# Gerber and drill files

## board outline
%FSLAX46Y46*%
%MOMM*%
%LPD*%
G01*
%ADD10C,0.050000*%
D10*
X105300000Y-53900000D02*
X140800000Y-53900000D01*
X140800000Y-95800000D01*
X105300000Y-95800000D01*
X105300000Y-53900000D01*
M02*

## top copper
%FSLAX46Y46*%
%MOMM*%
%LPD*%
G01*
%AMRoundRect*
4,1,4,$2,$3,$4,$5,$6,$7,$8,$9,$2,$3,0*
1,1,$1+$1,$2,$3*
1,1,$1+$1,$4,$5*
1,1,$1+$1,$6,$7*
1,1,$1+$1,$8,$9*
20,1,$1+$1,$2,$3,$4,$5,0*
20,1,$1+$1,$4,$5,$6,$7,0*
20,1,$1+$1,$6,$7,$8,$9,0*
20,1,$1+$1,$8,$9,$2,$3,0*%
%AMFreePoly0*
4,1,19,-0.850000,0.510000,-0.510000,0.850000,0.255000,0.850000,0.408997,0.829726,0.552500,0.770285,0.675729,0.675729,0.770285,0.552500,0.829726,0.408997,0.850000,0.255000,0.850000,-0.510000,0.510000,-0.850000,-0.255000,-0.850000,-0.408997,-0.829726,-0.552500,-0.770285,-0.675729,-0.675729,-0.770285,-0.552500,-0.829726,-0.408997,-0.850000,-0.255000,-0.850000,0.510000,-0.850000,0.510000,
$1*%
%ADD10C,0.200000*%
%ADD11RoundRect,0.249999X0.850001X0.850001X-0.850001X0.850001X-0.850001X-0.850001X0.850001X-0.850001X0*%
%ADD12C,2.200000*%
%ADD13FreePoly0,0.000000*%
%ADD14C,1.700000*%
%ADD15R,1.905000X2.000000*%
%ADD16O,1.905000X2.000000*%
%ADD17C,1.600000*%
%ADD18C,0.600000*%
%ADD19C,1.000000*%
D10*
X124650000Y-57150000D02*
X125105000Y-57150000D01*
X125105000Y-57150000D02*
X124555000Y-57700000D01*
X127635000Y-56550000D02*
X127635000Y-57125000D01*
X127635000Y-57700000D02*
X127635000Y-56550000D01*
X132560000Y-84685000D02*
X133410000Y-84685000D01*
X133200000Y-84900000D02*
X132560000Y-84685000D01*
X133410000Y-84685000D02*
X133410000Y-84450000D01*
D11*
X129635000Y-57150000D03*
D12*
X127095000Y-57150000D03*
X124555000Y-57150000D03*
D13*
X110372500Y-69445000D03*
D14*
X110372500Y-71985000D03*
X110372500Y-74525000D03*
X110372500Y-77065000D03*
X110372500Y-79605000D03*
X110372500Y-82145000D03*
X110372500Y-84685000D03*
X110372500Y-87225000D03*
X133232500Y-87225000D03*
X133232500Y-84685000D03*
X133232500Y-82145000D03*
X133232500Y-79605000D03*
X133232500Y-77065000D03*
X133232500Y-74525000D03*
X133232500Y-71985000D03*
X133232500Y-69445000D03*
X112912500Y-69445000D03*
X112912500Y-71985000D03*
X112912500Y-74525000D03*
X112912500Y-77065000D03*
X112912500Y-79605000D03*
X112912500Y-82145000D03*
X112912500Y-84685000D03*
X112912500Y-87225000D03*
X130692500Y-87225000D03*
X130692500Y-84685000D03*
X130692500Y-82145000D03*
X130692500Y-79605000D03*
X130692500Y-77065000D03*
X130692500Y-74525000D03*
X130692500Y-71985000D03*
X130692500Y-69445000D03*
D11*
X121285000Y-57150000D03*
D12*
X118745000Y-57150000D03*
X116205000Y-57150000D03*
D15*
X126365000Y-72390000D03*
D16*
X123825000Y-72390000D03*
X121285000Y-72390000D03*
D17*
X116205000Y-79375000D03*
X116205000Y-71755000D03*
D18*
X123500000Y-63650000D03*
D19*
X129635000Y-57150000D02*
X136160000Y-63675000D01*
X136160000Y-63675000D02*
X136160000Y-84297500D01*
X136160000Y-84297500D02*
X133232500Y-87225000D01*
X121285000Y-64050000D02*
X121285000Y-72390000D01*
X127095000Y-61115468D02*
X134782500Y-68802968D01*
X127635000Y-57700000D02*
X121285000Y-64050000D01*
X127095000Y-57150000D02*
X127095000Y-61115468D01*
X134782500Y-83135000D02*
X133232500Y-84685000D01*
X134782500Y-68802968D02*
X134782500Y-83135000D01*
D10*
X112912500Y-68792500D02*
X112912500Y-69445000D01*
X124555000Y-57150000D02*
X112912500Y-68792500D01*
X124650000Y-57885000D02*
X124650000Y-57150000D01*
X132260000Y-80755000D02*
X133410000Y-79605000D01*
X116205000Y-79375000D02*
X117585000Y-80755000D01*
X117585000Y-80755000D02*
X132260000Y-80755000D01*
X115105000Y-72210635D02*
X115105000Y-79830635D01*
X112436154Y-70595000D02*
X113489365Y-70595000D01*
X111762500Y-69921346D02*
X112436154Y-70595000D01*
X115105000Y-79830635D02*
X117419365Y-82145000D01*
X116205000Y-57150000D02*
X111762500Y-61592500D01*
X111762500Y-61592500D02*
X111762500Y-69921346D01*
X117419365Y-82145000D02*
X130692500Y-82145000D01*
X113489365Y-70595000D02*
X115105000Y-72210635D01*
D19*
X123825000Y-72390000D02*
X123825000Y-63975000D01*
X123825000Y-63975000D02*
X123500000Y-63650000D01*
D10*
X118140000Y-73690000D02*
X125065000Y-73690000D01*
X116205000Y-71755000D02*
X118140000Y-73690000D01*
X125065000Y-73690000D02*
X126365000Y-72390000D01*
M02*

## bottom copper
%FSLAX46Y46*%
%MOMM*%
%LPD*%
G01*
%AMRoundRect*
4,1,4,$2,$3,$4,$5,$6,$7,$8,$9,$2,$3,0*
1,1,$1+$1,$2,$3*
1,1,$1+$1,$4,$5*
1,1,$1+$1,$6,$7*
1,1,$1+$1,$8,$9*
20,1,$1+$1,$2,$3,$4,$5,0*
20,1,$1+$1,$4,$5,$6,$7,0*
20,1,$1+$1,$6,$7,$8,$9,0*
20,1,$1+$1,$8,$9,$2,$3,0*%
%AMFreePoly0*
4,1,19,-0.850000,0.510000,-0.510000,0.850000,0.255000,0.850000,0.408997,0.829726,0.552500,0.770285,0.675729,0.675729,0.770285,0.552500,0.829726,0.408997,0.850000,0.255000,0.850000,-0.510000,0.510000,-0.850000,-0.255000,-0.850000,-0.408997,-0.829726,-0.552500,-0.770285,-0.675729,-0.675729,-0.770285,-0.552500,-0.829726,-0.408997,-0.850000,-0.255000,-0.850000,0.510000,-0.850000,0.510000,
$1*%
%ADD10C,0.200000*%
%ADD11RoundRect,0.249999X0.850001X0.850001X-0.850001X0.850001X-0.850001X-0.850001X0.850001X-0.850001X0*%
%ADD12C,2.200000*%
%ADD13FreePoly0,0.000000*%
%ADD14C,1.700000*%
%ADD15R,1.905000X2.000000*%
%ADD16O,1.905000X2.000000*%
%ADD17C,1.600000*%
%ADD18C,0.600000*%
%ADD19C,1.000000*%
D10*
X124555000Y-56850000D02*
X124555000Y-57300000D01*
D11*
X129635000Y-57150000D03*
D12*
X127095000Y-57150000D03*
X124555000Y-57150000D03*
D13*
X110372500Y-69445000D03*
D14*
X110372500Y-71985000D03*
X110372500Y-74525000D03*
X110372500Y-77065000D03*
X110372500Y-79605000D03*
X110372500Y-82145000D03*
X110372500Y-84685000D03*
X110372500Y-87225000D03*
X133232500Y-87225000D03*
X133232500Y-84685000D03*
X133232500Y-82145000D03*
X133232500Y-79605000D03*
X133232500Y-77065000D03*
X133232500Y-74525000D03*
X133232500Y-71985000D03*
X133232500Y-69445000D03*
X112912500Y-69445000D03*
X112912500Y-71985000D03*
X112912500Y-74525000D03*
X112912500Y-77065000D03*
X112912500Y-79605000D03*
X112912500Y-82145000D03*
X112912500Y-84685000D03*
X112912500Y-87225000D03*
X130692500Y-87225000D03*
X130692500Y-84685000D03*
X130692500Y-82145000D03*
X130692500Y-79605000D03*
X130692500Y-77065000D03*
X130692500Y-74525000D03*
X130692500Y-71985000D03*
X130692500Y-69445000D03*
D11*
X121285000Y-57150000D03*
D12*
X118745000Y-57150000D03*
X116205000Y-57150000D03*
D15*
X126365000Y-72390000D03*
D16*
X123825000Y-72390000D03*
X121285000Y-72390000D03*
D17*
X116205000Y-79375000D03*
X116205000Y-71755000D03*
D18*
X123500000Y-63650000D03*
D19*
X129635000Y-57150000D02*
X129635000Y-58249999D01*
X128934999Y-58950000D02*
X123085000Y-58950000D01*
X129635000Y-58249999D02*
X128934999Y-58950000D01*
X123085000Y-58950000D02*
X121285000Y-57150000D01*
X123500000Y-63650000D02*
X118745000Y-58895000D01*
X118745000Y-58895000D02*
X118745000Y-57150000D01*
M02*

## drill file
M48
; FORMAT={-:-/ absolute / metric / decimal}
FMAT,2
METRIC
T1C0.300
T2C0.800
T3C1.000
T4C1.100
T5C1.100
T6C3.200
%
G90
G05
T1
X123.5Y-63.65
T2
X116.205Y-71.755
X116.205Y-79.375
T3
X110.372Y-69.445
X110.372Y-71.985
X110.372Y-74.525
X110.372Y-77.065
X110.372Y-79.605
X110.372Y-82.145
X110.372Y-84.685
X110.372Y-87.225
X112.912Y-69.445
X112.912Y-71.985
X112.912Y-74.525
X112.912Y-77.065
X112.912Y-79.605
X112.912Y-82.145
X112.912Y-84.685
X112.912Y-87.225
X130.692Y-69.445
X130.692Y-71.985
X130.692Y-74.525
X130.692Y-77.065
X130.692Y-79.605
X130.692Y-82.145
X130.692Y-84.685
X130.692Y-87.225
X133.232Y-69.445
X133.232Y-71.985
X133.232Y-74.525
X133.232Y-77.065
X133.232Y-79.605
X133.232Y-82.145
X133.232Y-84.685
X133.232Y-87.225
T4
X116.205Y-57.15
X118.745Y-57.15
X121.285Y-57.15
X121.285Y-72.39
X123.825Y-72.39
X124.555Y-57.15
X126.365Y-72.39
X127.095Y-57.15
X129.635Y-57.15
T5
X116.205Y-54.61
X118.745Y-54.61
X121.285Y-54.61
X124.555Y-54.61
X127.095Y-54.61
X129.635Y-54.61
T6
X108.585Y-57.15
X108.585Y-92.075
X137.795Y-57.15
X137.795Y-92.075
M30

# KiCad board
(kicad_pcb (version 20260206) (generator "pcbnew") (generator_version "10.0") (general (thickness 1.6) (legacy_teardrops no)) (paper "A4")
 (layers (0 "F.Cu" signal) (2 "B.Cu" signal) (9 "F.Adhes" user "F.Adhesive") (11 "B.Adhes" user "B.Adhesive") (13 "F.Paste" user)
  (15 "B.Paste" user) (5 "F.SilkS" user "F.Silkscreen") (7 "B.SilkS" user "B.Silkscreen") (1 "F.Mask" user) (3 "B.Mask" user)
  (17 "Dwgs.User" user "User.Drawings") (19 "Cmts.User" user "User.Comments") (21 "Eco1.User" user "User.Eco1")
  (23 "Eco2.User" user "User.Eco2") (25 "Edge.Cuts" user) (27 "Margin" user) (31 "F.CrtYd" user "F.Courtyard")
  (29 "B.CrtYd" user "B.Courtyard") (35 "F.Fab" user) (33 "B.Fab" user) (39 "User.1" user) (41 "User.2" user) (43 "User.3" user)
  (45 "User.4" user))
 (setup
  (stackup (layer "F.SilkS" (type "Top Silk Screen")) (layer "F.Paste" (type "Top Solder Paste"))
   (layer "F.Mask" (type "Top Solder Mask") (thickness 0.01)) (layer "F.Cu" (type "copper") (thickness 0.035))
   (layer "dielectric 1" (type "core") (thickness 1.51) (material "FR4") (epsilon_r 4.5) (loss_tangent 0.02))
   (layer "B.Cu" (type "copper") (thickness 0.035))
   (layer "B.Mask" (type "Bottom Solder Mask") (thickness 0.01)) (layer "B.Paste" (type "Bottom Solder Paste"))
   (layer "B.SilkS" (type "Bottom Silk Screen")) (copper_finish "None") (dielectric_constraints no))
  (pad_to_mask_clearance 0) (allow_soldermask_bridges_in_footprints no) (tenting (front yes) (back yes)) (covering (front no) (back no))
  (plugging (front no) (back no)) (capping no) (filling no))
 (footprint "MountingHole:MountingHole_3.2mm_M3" (layer "F.Cu") (at 108.585 92.075)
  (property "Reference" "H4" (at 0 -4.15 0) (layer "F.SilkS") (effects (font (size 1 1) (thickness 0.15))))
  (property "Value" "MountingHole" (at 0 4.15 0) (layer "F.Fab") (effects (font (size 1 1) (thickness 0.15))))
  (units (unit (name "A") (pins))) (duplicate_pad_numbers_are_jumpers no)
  (pad "" np_thru_hole circle (at 0 0) (size 3.2 3.2) (drill 3.2) (layers "*.Cu" "*.Mask")))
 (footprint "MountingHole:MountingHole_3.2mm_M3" (layer "F.Cu") (at 108.585 57.15)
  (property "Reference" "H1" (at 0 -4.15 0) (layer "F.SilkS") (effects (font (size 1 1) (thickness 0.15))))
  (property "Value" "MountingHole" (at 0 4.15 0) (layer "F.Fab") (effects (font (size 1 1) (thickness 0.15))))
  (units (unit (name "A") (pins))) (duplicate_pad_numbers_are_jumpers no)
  (pad "" np_thru_hole circle (at 0 0) (size 3.2 3.2) (drill 3.2) (layers "*.Cu" "*.Mask")))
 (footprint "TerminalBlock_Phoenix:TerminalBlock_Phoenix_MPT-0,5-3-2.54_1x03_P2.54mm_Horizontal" (layer "F.Cu") (at 129.635 57.15 180)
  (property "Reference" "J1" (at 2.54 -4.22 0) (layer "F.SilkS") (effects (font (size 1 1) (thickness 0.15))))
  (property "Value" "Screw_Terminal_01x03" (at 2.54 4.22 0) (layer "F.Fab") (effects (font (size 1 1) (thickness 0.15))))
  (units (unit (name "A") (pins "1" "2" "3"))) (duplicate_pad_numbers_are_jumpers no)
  (pad "" np_thru_hole circle (at 0 2.54 180) (size 1.1 1.1) (drill 1.1) (layers "*.Cu" "*.Mask"))
  (pad "" np_thru_hole circle (at 2.54 2.54 180) (size 1.1 1.1) (drill 1.1) (layers "*.Cu" "*.Mask"))
  (pad "" np_thru_hole circle (at 5.08 2.54 180) (size 1.1 1.1) (drill 1.1) (layers "*.Cu" "*.Mask"))
  (pad "1" thru_hole roundrect (at 0 0 180) (size 2.2 2.2) (drill 1.1) (layers "*.Cu" "*.Mask") (remove_unused_layers no)
   (roundrect_rratio 0.113636) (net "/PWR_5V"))
  (pad "2" thru_hole circle (at 2.54 0 180) (size 2.2 2.2) (drill 1.1) (layers "*.Cu" "*.Mask") (remove_unused_layers no) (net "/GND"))
  (pad "3" thru_hole circle (at 5.08 0 180) (size 2.2 2.2) (drill 1.1) (layers "*.Cu" "*.Mask") (remove_unused_layers no)
   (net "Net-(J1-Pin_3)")))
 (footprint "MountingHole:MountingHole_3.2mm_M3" (layer "F.Cu") (at 137.795 57.15)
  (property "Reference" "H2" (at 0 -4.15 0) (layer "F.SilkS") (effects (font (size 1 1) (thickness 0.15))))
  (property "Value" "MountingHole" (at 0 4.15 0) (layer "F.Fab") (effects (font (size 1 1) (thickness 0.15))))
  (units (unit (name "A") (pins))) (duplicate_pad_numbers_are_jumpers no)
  (pad "" np_thru_hole circle (at 0 0) (size 3.2 3.2) (drill 3.2) (layers "*.Cu" "*.Mask")))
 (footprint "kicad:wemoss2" (layer "F.Cu") (at 110.3725 69.445)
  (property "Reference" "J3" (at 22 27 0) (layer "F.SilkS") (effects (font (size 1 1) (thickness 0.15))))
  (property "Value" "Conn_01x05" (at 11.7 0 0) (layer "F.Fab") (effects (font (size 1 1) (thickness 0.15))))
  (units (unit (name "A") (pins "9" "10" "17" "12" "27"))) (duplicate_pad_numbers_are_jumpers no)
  (pad "1" thru_hole roundrect (at 0 0) (size 1.7 1.7) (drill 1) (layers "*.Cu" "*.Mask") (remove_unused_layers no) (roundrect_rratio 0.35)
   (chamfer_ratio 0.2) (chamfer top_left bottom_right))
  (pad "2" thru_hole circle (at 0 2.54) (size 1.7 1.7) (drill 1) (layers "*.Cu" "*.Mask") (remove_unused_layers no))
  (pad "3" thru_hole circle (at 0 5.08) (size 1.7 1.7) (drill 1) (layers "*.Cu" "*.Mask") (remove_unused_layers no))
  (pad "4" thru_hole circle (at 0 7.62) (size 1.7 1.7) (drill 1) (layers "*.Cu" "*.Mask") (remove_unused_layers no))
  (pad "5" thru_hole circle (at 0 10.16) (size 1.7 1.7) (drill 1) (layers "*.Cu" "*.Mask") (remove_unused_layers no))
  (pad "6" thru_hole circle (at 0 12.7) (size 1.7 1.7) (drill 1) (layers "*.Cu" "*.Mask") (remove_unused_layers no))
  (pad "7" thru_hole circle (at 0 15.24) (size 1.7 1.7) (drill 1) (layers "*.Cu" "*.Mask") (remove_unused_layers no))
  (pad "8" thru_hole circle (at 0 17.78) (size 1.7 1.7) (drill 1) (layers "*.Cu" "*.Mask") (remove_unused_layers no))
  (pad "9" thru_hole circle (at 22.86 17.78) (size 1.7 1.7) (drill 1) (layers "*.Cu" "*.Mask") (remove_unused_layers no) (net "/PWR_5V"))
  (pad "10" thru_hole circle (at 22.86 15.24) (size 1.7 1.7) (drill 1) (layers "*.Cu" "*.Mask") (remove_unused_layers no) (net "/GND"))
  (pad "11" thru_hole circle (at 22.86 12.7) (size 1.7 1.7) (drill 1) (layers "*.Cu" "*.Mask") (remove_unused_layers no))
  (pad "12" thru_hole circle (at 22.86 10.16) (size 1.7 1.7) (drill 1) (layers "*.Cu" "*.Mask") (remove_unused_layers no) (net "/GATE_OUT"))
  (pad "13" thru_hole circle (at 22.86 7.62) (size 1.7 1.7) (drill 1) (layers "*.Cu" "*.Mask") (remove_unused_layers no))
  (pad "14" thru_hole circle (at 22.86 5.08) (size 1.7 1.7) (drill 1) (layers "*.Cu" "*.Mask") (remove_unused_layers no))
  (pad "15" thru_hole circle (at 22.86 2.54) (size 1.7 1.7) (drill 1) (layers "*.Cu" "*.Mask") (remove_unused_layers no))
  (pad "16" thru_hole circle (at 22.86 0) (size 1.7 1.7) (drill 1) (layers "*.Cu" "*.Mask") (remove_unused_layers no))
  (pad "17" thru_hole circle (at 2.54 0) (size 1.7 1.7) (drill 1) (layers "*.Cu" "*.Mask") (remove_unused_layers no) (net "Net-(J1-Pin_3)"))
  (pad "18" thru_hole circle (at 2.54 2.54) (size 1.7 1.7) (drill 1) (layers "*.Cu" "*.Mask") (remove_unused_layers no))
  (pad "19" thru_hole circle (at 2.54 5.08) (size 1.7 1.7) (drill 1) (layers "*.Cu" "*.Mask") (remove_unused_layers no))
  (pad "20" thru_hole circle (at 2.54 7.62) (size 1.7 1.7) (drill 1) (layers "*.Cu" "*.Mask") (remove_unused_layers no))
  (pad "21" thru_hole circle (at 2.54 10.16) (size 1.7 1.7) (drill 1) (layers "*.Cu" "*.Mask") (remove_unused_layers no))
  (pad "22" thru_hole circle (at 2.54 12.7) (size 1.7 1.7) (drill 1) (layers "*.Cu" "*.Mask") (remove_unused_layers no))
  (pad "23" thru_hole circle (at 2.54 15.24) (size 1.7 1.7) (drill 1) (layers "*.Cu" "*.Mask") (remove_unused_layers no))
  (pad "24" thru_hole circle (at 2.54 17.78) (size 1.7 1.7) (drill 1) (layers "*.Cu" "*.Mask") (remove_unused_layers no))
  (pad "25" thru_hole circle (at 20.32 17.78) (size 1.7 1.7) (drill 1) (layers "*.Cu" "*.Mask") (remove_unused_layers no))
  (pad "26" thru_hole circle (at 20.32 15.24) (size 1.7 1.7) (drill 1) (layers "*.Cu" "*.Mask") (remove_unused_layers no))
  (pad "27" thru_hole circle (at 20.32 12.7) (size 1.7 1.7) (drill 1) (layers "*.Cu" "*.Mask") (remove_unused_layers no)
   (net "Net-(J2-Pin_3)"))
  (pad "28" thru_hole circle (at 20.32 10.16) (size 1.7 1.7) (drill 1) (layers "*.Cu" "*.Mask") (remove_unused_layers no))
  (pad "29" thru_hole circle (at 20.32 7.62) (size 1.7 1.7) (drill 1) (layers "*.Cu" "*.Mask") (remove_unused_layers no))
  (pad "30" thru_hole circle (at 20.32 5.08) (size 1.7 1.7) (drill 1) (layers "*.Cu" "*.Mask") (remove_unused_layers no))
  (pad "31" thru_hole circle (at 20.32 2.54) (size 1.7 1.7) (drill 1) (layers "*.Cu" "*.Mask") (remove_unused_layers no))
  (pad "32" thru_hole circle (at 20.32 0) (size 1.7 1.7) (drill 1) (layers "*.Cu" "*.Mask") (remove_unused_layers no)))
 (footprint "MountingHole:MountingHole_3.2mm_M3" (layer "F.Cu") (at 137.795 92.075)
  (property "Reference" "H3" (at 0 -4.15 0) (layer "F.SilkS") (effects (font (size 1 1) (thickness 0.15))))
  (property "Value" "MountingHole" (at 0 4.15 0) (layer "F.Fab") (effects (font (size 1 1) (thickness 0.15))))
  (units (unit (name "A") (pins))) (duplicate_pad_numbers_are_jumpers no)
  (pad "" np_thru_hole circle (at 0 0) (size 3.2 3.2) (drill 3.2) (layers "*.Cu" "*.Mask")))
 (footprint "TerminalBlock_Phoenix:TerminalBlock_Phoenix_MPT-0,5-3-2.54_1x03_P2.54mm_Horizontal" (layer "F.Cu") (at 121.285 57.15 180)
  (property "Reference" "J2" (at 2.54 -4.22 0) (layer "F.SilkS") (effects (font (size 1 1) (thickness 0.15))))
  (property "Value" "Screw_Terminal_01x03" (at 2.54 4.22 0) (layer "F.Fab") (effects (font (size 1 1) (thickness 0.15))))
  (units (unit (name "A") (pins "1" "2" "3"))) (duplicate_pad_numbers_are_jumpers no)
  (pad "" np_thru_hole circle (at 0 2.54 180) (size 1.1 1.1) (drill 1.1) (layers "*.Cu" "*.Mask"))
  (pad "" np_thru_hole circle (at 2.54 2.54 180) (size 1.1 1.1) (drill 1.1) (layers "*.Cu" "*.Mask"))
  (pad "" np_thru_hole circle (at 5.08 2.54 180) (size 1.1 1.1) (drill 1.1) (layers "*.Cu" "*.Mask"))
  (pad "1" thru_hole roundrect (at 0 0 180) (size 2.2 2.2) (drill 1.1) (layers "*.Cu" "*.Mask") (remove_unused_layers no)
   (roundrect_rratio 0.113636) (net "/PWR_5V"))
  (pad "2" thru_hole circle (at 2.54 0 180) (size 2.2 2.2) (drill 1.1) (layers "*.Cu" "*.Mask") (remove_unused_layers no) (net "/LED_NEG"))
  (pad "3" thru_hole circle (at 5.08 0 180) (size 2.2 2.2) (drill 1.1) (layers "*.Cu" "*.Mask") (remove_unused_layers no)
   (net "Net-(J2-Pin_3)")))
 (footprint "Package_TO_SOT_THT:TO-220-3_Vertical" (layer "B.Cu") (at 126.365 72.39 180)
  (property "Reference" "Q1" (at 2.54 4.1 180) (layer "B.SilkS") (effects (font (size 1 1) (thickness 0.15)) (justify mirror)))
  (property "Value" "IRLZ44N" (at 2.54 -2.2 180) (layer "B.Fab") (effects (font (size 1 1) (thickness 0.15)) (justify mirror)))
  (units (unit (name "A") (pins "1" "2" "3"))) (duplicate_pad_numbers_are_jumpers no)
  (pad "1" thru_hole rect (at 0 0 180) (size 1.905 2) (drill 1.1) (layers "*.Cu" "*.Mask") (remove_unused_layers no) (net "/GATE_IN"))
  (pad "2" thru_hole oval (at 2.54 0 180) (size 1.905 2) (drill 1.1) (layers "*.Cu" "*.Mask") (remove_unused_layers no) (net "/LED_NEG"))
  (pad "3" thru_hole oval (at 5.08 0 180) (size 1.905 2) (drill 1.1) (layers "*.Cu" "*.Mask") (remove_unused_layers no) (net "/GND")))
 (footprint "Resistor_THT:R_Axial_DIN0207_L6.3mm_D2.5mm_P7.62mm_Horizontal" (layer "B.Cu") (at 116.205 79.375 90)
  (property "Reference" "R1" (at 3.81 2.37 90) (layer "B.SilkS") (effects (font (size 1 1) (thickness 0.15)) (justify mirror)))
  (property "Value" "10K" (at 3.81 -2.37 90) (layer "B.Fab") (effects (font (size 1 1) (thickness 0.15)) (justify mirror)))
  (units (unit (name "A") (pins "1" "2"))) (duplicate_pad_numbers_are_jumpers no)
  (pad "1" thru_hole circle (at 0 0 90) (size 1.6 1.6) (drill 0.8) (layers "*.Cu" "*.Mask") (remove_unused_layers no) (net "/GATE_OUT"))
  (pad "2" thru_hole circle (at 7.62 0 90) (size 1.6 1.6) (drill 0.8) (layers "*.Cu" "*.Mask") (remove_unused_layers no) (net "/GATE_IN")))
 (gr_line (start 124.65 57.15) (end 125.105 57.15) (stroke (width 0.2) (type default)) (layer "F.Cu") (net "Net-(J1-Pin_3)"))
 (gr_line (start 125.105 57.15) (end 124.555 57.7) (stroke (width 0.2) (type default)) (layer "F.Cu") (net "Net-(J1-Pin_3)"))
 (gr_line (start 127.635 56.55) (end 127.635 57.125) (stroke (width 0.2) (type default)) (layer "F.Cu") (net "/GND"))
 (gr_line (start 127.635 57.7) (end 127.635 56.55) (stroke (width 0.2) (type default)) (layer "F.Cu") (net "/GND"))
 (gr_line (start 132.56 84.685) (end 133.41 84.685) (stroke (width 0.2) (type default)) (layer "F.Cu") (net "/GND"))
 (gr_line (start 133.2 84.9) (end 132.56 84.685) (stroke (width 0.2) (type default)) (layer "F.Cu") (net "/GND"))
 (gr_line (start 133.41 84.685) (end 133.41 84.45) (stroke (width 0.2) (type default)) (layer "F.Cu") (net "/GND"))
 (gr_line (start 124.555 56.85) (end 124.555 57.3) (stroke (width 0.2) (type default)) (layer "B.Cu") (net "Net-(J1-Pin_3)"))
 (gr_rect (start 105.3 53.9) (end 140.8 95.8) (stroke (width 0.05) (type default)) (fill no) (layer "Edge.Cuts"))
 (segment (start 129.635 57.15) (end 136.16 63.675) (width 1) (layer "F.Cu") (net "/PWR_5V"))
 (segment (start 136.16 63.675) (end 136.16 84.2975) (width 1) (layer "F.Cu") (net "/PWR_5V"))
 (segment (start 136.16 84.2975) (end 133.2325 87.225) (width 1) (layer "F.Cu") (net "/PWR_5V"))
 (segment (start 129.635 57.15) (end 129.635 58.249999) (width 1) (layer "B.Cu") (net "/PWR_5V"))
 (segment (start 128.934999 58.95) (end 123.085 58.95) (width 1) (layer "B.Cu") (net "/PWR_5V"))
 (segment (start 129.635 58.249999) (end 128.934999 58.95) (width 1) (layer "B.Cu") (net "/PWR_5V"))
 (segment (start 123.085 58.95) (end 121.285 57.15) (width 1) (layer "B.Cu") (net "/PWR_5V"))
 (segment (start 121.285 64.05) (end 121.285 72.39) (width 1) (layer "F.Cu") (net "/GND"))
 (segment (start 127.095 61.115468) (end 134.7825 68.802968) (width 1) (layer "F.Cu") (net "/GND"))
 (segment (start 127.635 57.7) (end 121.285 64.05) (width 1) (layer "F.Cu") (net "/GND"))
 (segment (start 127.095 57.15) (end 127.095 61.115468) (width 1) (layer "F.Cu") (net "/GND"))
 (segment (start 134.7825 83.135) (end 133.2325 84.685) (width 1) (layer "F.Cu") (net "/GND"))
 (segment (start 134.7825 68.802968) (end 134.7825 83.135) (width 1) (layer "F.Cu") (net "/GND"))
 (segment (start 112.9125 68.7925) (end 112.9125 69.445) (width 0.2) (layer "F.Cu") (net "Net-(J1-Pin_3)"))
 (segment (start 124.555 57.15) (end 112.9125 68.7925) (width 0.2) (layer "F.Cu") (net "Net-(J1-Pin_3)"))
 (segment (start 124.65 57.885) (end 124.65 57.15) (width 0.2) (layer "F.Cu") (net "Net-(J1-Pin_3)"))
 (segment (start 132.26 80.755) (end 133.41 79.605) (width 0.2) (layer "F.Cu") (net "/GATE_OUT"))
 (segment (start 116.205 79.375) (end 117.585 80.755) (width 0.2) (layer "F.Cu") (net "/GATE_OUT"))
 (segment (start 117.585 80.755) (end 132.26 80.755) (width 0.2) (layer "F.Cu") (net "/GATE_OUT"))
 (segment (start 115.105 72.210635) (end 115.105 79.830635) (width 0.2) (layer "F.Cu") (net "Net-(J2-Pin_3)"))
 (segment (start 112.436154 70.595) (end 113.489365 70.595) (width 0.2) (layer "F.Cu") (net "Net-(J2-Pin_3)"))
 (segment (start 111.7625 69.921346) (end 112.436154 70.595) (width 0.2) (layer "F.Cu") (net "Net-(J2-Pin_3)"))
 (segment (start 115.105 79.830635) (end 117.419365 82.145) (width 0.2) (layer "F.Cu") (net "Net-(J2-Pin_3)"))
 (segment (start 116.205 57.15) (end 111.7625 61.5925) (width 0.2) (layer "F.Cu") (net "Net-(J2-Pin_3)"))
 (segment (start 111.7625 61.5925) (end 111.7625 69.921346) (width 0.2) (layer "F.Cu") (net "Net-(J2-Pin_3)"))
 (segment (start 117.419365 82.145) (end 130.6925 82.145) (width 0.2) (layer "F.Cu") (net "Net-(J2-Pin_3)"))
 (segment (start 113.489365 70.595) (end 115.105 72.210635) (width 0.2) (layer "F.Cu") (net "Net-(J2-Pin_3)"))
 (segment (start 123.825 72.39) (end 123.825 63.975) (width 1) (layer "F.Cu") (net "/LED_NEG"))
 (segment (start 123.825 63.975) (end 123.5 63.65) (width 1) (layer "F.Cu") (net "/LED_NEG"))
 (via (at 123.5 63.65) (size 0.6) (drill 0.3) (layers "F.Cu" "B.Cu") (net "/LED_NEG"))
 (segment (start 123.5 63.65) (end 118.745 58.895) (width 1) (layer "B.Cu") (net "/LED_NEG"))
 (segment (start 118.745 58.895) (end 118.745 57.15) (width 1) (layer "B.Cu") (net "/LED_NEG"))
 (segment (start 118.14 73.69) (end 125.065 73.69) (width 0.2) (layer "F.Cu") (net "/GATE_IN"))
 (segment (start 116.205 71.755) (end 118.14 73.69) (width 0.2) (layer "F.Cu") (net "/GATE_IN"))
 (segment (start 125.065 73.69) (end 126.365 72.39) (width 0.2) (layer "F.Cu") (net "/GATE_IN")))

